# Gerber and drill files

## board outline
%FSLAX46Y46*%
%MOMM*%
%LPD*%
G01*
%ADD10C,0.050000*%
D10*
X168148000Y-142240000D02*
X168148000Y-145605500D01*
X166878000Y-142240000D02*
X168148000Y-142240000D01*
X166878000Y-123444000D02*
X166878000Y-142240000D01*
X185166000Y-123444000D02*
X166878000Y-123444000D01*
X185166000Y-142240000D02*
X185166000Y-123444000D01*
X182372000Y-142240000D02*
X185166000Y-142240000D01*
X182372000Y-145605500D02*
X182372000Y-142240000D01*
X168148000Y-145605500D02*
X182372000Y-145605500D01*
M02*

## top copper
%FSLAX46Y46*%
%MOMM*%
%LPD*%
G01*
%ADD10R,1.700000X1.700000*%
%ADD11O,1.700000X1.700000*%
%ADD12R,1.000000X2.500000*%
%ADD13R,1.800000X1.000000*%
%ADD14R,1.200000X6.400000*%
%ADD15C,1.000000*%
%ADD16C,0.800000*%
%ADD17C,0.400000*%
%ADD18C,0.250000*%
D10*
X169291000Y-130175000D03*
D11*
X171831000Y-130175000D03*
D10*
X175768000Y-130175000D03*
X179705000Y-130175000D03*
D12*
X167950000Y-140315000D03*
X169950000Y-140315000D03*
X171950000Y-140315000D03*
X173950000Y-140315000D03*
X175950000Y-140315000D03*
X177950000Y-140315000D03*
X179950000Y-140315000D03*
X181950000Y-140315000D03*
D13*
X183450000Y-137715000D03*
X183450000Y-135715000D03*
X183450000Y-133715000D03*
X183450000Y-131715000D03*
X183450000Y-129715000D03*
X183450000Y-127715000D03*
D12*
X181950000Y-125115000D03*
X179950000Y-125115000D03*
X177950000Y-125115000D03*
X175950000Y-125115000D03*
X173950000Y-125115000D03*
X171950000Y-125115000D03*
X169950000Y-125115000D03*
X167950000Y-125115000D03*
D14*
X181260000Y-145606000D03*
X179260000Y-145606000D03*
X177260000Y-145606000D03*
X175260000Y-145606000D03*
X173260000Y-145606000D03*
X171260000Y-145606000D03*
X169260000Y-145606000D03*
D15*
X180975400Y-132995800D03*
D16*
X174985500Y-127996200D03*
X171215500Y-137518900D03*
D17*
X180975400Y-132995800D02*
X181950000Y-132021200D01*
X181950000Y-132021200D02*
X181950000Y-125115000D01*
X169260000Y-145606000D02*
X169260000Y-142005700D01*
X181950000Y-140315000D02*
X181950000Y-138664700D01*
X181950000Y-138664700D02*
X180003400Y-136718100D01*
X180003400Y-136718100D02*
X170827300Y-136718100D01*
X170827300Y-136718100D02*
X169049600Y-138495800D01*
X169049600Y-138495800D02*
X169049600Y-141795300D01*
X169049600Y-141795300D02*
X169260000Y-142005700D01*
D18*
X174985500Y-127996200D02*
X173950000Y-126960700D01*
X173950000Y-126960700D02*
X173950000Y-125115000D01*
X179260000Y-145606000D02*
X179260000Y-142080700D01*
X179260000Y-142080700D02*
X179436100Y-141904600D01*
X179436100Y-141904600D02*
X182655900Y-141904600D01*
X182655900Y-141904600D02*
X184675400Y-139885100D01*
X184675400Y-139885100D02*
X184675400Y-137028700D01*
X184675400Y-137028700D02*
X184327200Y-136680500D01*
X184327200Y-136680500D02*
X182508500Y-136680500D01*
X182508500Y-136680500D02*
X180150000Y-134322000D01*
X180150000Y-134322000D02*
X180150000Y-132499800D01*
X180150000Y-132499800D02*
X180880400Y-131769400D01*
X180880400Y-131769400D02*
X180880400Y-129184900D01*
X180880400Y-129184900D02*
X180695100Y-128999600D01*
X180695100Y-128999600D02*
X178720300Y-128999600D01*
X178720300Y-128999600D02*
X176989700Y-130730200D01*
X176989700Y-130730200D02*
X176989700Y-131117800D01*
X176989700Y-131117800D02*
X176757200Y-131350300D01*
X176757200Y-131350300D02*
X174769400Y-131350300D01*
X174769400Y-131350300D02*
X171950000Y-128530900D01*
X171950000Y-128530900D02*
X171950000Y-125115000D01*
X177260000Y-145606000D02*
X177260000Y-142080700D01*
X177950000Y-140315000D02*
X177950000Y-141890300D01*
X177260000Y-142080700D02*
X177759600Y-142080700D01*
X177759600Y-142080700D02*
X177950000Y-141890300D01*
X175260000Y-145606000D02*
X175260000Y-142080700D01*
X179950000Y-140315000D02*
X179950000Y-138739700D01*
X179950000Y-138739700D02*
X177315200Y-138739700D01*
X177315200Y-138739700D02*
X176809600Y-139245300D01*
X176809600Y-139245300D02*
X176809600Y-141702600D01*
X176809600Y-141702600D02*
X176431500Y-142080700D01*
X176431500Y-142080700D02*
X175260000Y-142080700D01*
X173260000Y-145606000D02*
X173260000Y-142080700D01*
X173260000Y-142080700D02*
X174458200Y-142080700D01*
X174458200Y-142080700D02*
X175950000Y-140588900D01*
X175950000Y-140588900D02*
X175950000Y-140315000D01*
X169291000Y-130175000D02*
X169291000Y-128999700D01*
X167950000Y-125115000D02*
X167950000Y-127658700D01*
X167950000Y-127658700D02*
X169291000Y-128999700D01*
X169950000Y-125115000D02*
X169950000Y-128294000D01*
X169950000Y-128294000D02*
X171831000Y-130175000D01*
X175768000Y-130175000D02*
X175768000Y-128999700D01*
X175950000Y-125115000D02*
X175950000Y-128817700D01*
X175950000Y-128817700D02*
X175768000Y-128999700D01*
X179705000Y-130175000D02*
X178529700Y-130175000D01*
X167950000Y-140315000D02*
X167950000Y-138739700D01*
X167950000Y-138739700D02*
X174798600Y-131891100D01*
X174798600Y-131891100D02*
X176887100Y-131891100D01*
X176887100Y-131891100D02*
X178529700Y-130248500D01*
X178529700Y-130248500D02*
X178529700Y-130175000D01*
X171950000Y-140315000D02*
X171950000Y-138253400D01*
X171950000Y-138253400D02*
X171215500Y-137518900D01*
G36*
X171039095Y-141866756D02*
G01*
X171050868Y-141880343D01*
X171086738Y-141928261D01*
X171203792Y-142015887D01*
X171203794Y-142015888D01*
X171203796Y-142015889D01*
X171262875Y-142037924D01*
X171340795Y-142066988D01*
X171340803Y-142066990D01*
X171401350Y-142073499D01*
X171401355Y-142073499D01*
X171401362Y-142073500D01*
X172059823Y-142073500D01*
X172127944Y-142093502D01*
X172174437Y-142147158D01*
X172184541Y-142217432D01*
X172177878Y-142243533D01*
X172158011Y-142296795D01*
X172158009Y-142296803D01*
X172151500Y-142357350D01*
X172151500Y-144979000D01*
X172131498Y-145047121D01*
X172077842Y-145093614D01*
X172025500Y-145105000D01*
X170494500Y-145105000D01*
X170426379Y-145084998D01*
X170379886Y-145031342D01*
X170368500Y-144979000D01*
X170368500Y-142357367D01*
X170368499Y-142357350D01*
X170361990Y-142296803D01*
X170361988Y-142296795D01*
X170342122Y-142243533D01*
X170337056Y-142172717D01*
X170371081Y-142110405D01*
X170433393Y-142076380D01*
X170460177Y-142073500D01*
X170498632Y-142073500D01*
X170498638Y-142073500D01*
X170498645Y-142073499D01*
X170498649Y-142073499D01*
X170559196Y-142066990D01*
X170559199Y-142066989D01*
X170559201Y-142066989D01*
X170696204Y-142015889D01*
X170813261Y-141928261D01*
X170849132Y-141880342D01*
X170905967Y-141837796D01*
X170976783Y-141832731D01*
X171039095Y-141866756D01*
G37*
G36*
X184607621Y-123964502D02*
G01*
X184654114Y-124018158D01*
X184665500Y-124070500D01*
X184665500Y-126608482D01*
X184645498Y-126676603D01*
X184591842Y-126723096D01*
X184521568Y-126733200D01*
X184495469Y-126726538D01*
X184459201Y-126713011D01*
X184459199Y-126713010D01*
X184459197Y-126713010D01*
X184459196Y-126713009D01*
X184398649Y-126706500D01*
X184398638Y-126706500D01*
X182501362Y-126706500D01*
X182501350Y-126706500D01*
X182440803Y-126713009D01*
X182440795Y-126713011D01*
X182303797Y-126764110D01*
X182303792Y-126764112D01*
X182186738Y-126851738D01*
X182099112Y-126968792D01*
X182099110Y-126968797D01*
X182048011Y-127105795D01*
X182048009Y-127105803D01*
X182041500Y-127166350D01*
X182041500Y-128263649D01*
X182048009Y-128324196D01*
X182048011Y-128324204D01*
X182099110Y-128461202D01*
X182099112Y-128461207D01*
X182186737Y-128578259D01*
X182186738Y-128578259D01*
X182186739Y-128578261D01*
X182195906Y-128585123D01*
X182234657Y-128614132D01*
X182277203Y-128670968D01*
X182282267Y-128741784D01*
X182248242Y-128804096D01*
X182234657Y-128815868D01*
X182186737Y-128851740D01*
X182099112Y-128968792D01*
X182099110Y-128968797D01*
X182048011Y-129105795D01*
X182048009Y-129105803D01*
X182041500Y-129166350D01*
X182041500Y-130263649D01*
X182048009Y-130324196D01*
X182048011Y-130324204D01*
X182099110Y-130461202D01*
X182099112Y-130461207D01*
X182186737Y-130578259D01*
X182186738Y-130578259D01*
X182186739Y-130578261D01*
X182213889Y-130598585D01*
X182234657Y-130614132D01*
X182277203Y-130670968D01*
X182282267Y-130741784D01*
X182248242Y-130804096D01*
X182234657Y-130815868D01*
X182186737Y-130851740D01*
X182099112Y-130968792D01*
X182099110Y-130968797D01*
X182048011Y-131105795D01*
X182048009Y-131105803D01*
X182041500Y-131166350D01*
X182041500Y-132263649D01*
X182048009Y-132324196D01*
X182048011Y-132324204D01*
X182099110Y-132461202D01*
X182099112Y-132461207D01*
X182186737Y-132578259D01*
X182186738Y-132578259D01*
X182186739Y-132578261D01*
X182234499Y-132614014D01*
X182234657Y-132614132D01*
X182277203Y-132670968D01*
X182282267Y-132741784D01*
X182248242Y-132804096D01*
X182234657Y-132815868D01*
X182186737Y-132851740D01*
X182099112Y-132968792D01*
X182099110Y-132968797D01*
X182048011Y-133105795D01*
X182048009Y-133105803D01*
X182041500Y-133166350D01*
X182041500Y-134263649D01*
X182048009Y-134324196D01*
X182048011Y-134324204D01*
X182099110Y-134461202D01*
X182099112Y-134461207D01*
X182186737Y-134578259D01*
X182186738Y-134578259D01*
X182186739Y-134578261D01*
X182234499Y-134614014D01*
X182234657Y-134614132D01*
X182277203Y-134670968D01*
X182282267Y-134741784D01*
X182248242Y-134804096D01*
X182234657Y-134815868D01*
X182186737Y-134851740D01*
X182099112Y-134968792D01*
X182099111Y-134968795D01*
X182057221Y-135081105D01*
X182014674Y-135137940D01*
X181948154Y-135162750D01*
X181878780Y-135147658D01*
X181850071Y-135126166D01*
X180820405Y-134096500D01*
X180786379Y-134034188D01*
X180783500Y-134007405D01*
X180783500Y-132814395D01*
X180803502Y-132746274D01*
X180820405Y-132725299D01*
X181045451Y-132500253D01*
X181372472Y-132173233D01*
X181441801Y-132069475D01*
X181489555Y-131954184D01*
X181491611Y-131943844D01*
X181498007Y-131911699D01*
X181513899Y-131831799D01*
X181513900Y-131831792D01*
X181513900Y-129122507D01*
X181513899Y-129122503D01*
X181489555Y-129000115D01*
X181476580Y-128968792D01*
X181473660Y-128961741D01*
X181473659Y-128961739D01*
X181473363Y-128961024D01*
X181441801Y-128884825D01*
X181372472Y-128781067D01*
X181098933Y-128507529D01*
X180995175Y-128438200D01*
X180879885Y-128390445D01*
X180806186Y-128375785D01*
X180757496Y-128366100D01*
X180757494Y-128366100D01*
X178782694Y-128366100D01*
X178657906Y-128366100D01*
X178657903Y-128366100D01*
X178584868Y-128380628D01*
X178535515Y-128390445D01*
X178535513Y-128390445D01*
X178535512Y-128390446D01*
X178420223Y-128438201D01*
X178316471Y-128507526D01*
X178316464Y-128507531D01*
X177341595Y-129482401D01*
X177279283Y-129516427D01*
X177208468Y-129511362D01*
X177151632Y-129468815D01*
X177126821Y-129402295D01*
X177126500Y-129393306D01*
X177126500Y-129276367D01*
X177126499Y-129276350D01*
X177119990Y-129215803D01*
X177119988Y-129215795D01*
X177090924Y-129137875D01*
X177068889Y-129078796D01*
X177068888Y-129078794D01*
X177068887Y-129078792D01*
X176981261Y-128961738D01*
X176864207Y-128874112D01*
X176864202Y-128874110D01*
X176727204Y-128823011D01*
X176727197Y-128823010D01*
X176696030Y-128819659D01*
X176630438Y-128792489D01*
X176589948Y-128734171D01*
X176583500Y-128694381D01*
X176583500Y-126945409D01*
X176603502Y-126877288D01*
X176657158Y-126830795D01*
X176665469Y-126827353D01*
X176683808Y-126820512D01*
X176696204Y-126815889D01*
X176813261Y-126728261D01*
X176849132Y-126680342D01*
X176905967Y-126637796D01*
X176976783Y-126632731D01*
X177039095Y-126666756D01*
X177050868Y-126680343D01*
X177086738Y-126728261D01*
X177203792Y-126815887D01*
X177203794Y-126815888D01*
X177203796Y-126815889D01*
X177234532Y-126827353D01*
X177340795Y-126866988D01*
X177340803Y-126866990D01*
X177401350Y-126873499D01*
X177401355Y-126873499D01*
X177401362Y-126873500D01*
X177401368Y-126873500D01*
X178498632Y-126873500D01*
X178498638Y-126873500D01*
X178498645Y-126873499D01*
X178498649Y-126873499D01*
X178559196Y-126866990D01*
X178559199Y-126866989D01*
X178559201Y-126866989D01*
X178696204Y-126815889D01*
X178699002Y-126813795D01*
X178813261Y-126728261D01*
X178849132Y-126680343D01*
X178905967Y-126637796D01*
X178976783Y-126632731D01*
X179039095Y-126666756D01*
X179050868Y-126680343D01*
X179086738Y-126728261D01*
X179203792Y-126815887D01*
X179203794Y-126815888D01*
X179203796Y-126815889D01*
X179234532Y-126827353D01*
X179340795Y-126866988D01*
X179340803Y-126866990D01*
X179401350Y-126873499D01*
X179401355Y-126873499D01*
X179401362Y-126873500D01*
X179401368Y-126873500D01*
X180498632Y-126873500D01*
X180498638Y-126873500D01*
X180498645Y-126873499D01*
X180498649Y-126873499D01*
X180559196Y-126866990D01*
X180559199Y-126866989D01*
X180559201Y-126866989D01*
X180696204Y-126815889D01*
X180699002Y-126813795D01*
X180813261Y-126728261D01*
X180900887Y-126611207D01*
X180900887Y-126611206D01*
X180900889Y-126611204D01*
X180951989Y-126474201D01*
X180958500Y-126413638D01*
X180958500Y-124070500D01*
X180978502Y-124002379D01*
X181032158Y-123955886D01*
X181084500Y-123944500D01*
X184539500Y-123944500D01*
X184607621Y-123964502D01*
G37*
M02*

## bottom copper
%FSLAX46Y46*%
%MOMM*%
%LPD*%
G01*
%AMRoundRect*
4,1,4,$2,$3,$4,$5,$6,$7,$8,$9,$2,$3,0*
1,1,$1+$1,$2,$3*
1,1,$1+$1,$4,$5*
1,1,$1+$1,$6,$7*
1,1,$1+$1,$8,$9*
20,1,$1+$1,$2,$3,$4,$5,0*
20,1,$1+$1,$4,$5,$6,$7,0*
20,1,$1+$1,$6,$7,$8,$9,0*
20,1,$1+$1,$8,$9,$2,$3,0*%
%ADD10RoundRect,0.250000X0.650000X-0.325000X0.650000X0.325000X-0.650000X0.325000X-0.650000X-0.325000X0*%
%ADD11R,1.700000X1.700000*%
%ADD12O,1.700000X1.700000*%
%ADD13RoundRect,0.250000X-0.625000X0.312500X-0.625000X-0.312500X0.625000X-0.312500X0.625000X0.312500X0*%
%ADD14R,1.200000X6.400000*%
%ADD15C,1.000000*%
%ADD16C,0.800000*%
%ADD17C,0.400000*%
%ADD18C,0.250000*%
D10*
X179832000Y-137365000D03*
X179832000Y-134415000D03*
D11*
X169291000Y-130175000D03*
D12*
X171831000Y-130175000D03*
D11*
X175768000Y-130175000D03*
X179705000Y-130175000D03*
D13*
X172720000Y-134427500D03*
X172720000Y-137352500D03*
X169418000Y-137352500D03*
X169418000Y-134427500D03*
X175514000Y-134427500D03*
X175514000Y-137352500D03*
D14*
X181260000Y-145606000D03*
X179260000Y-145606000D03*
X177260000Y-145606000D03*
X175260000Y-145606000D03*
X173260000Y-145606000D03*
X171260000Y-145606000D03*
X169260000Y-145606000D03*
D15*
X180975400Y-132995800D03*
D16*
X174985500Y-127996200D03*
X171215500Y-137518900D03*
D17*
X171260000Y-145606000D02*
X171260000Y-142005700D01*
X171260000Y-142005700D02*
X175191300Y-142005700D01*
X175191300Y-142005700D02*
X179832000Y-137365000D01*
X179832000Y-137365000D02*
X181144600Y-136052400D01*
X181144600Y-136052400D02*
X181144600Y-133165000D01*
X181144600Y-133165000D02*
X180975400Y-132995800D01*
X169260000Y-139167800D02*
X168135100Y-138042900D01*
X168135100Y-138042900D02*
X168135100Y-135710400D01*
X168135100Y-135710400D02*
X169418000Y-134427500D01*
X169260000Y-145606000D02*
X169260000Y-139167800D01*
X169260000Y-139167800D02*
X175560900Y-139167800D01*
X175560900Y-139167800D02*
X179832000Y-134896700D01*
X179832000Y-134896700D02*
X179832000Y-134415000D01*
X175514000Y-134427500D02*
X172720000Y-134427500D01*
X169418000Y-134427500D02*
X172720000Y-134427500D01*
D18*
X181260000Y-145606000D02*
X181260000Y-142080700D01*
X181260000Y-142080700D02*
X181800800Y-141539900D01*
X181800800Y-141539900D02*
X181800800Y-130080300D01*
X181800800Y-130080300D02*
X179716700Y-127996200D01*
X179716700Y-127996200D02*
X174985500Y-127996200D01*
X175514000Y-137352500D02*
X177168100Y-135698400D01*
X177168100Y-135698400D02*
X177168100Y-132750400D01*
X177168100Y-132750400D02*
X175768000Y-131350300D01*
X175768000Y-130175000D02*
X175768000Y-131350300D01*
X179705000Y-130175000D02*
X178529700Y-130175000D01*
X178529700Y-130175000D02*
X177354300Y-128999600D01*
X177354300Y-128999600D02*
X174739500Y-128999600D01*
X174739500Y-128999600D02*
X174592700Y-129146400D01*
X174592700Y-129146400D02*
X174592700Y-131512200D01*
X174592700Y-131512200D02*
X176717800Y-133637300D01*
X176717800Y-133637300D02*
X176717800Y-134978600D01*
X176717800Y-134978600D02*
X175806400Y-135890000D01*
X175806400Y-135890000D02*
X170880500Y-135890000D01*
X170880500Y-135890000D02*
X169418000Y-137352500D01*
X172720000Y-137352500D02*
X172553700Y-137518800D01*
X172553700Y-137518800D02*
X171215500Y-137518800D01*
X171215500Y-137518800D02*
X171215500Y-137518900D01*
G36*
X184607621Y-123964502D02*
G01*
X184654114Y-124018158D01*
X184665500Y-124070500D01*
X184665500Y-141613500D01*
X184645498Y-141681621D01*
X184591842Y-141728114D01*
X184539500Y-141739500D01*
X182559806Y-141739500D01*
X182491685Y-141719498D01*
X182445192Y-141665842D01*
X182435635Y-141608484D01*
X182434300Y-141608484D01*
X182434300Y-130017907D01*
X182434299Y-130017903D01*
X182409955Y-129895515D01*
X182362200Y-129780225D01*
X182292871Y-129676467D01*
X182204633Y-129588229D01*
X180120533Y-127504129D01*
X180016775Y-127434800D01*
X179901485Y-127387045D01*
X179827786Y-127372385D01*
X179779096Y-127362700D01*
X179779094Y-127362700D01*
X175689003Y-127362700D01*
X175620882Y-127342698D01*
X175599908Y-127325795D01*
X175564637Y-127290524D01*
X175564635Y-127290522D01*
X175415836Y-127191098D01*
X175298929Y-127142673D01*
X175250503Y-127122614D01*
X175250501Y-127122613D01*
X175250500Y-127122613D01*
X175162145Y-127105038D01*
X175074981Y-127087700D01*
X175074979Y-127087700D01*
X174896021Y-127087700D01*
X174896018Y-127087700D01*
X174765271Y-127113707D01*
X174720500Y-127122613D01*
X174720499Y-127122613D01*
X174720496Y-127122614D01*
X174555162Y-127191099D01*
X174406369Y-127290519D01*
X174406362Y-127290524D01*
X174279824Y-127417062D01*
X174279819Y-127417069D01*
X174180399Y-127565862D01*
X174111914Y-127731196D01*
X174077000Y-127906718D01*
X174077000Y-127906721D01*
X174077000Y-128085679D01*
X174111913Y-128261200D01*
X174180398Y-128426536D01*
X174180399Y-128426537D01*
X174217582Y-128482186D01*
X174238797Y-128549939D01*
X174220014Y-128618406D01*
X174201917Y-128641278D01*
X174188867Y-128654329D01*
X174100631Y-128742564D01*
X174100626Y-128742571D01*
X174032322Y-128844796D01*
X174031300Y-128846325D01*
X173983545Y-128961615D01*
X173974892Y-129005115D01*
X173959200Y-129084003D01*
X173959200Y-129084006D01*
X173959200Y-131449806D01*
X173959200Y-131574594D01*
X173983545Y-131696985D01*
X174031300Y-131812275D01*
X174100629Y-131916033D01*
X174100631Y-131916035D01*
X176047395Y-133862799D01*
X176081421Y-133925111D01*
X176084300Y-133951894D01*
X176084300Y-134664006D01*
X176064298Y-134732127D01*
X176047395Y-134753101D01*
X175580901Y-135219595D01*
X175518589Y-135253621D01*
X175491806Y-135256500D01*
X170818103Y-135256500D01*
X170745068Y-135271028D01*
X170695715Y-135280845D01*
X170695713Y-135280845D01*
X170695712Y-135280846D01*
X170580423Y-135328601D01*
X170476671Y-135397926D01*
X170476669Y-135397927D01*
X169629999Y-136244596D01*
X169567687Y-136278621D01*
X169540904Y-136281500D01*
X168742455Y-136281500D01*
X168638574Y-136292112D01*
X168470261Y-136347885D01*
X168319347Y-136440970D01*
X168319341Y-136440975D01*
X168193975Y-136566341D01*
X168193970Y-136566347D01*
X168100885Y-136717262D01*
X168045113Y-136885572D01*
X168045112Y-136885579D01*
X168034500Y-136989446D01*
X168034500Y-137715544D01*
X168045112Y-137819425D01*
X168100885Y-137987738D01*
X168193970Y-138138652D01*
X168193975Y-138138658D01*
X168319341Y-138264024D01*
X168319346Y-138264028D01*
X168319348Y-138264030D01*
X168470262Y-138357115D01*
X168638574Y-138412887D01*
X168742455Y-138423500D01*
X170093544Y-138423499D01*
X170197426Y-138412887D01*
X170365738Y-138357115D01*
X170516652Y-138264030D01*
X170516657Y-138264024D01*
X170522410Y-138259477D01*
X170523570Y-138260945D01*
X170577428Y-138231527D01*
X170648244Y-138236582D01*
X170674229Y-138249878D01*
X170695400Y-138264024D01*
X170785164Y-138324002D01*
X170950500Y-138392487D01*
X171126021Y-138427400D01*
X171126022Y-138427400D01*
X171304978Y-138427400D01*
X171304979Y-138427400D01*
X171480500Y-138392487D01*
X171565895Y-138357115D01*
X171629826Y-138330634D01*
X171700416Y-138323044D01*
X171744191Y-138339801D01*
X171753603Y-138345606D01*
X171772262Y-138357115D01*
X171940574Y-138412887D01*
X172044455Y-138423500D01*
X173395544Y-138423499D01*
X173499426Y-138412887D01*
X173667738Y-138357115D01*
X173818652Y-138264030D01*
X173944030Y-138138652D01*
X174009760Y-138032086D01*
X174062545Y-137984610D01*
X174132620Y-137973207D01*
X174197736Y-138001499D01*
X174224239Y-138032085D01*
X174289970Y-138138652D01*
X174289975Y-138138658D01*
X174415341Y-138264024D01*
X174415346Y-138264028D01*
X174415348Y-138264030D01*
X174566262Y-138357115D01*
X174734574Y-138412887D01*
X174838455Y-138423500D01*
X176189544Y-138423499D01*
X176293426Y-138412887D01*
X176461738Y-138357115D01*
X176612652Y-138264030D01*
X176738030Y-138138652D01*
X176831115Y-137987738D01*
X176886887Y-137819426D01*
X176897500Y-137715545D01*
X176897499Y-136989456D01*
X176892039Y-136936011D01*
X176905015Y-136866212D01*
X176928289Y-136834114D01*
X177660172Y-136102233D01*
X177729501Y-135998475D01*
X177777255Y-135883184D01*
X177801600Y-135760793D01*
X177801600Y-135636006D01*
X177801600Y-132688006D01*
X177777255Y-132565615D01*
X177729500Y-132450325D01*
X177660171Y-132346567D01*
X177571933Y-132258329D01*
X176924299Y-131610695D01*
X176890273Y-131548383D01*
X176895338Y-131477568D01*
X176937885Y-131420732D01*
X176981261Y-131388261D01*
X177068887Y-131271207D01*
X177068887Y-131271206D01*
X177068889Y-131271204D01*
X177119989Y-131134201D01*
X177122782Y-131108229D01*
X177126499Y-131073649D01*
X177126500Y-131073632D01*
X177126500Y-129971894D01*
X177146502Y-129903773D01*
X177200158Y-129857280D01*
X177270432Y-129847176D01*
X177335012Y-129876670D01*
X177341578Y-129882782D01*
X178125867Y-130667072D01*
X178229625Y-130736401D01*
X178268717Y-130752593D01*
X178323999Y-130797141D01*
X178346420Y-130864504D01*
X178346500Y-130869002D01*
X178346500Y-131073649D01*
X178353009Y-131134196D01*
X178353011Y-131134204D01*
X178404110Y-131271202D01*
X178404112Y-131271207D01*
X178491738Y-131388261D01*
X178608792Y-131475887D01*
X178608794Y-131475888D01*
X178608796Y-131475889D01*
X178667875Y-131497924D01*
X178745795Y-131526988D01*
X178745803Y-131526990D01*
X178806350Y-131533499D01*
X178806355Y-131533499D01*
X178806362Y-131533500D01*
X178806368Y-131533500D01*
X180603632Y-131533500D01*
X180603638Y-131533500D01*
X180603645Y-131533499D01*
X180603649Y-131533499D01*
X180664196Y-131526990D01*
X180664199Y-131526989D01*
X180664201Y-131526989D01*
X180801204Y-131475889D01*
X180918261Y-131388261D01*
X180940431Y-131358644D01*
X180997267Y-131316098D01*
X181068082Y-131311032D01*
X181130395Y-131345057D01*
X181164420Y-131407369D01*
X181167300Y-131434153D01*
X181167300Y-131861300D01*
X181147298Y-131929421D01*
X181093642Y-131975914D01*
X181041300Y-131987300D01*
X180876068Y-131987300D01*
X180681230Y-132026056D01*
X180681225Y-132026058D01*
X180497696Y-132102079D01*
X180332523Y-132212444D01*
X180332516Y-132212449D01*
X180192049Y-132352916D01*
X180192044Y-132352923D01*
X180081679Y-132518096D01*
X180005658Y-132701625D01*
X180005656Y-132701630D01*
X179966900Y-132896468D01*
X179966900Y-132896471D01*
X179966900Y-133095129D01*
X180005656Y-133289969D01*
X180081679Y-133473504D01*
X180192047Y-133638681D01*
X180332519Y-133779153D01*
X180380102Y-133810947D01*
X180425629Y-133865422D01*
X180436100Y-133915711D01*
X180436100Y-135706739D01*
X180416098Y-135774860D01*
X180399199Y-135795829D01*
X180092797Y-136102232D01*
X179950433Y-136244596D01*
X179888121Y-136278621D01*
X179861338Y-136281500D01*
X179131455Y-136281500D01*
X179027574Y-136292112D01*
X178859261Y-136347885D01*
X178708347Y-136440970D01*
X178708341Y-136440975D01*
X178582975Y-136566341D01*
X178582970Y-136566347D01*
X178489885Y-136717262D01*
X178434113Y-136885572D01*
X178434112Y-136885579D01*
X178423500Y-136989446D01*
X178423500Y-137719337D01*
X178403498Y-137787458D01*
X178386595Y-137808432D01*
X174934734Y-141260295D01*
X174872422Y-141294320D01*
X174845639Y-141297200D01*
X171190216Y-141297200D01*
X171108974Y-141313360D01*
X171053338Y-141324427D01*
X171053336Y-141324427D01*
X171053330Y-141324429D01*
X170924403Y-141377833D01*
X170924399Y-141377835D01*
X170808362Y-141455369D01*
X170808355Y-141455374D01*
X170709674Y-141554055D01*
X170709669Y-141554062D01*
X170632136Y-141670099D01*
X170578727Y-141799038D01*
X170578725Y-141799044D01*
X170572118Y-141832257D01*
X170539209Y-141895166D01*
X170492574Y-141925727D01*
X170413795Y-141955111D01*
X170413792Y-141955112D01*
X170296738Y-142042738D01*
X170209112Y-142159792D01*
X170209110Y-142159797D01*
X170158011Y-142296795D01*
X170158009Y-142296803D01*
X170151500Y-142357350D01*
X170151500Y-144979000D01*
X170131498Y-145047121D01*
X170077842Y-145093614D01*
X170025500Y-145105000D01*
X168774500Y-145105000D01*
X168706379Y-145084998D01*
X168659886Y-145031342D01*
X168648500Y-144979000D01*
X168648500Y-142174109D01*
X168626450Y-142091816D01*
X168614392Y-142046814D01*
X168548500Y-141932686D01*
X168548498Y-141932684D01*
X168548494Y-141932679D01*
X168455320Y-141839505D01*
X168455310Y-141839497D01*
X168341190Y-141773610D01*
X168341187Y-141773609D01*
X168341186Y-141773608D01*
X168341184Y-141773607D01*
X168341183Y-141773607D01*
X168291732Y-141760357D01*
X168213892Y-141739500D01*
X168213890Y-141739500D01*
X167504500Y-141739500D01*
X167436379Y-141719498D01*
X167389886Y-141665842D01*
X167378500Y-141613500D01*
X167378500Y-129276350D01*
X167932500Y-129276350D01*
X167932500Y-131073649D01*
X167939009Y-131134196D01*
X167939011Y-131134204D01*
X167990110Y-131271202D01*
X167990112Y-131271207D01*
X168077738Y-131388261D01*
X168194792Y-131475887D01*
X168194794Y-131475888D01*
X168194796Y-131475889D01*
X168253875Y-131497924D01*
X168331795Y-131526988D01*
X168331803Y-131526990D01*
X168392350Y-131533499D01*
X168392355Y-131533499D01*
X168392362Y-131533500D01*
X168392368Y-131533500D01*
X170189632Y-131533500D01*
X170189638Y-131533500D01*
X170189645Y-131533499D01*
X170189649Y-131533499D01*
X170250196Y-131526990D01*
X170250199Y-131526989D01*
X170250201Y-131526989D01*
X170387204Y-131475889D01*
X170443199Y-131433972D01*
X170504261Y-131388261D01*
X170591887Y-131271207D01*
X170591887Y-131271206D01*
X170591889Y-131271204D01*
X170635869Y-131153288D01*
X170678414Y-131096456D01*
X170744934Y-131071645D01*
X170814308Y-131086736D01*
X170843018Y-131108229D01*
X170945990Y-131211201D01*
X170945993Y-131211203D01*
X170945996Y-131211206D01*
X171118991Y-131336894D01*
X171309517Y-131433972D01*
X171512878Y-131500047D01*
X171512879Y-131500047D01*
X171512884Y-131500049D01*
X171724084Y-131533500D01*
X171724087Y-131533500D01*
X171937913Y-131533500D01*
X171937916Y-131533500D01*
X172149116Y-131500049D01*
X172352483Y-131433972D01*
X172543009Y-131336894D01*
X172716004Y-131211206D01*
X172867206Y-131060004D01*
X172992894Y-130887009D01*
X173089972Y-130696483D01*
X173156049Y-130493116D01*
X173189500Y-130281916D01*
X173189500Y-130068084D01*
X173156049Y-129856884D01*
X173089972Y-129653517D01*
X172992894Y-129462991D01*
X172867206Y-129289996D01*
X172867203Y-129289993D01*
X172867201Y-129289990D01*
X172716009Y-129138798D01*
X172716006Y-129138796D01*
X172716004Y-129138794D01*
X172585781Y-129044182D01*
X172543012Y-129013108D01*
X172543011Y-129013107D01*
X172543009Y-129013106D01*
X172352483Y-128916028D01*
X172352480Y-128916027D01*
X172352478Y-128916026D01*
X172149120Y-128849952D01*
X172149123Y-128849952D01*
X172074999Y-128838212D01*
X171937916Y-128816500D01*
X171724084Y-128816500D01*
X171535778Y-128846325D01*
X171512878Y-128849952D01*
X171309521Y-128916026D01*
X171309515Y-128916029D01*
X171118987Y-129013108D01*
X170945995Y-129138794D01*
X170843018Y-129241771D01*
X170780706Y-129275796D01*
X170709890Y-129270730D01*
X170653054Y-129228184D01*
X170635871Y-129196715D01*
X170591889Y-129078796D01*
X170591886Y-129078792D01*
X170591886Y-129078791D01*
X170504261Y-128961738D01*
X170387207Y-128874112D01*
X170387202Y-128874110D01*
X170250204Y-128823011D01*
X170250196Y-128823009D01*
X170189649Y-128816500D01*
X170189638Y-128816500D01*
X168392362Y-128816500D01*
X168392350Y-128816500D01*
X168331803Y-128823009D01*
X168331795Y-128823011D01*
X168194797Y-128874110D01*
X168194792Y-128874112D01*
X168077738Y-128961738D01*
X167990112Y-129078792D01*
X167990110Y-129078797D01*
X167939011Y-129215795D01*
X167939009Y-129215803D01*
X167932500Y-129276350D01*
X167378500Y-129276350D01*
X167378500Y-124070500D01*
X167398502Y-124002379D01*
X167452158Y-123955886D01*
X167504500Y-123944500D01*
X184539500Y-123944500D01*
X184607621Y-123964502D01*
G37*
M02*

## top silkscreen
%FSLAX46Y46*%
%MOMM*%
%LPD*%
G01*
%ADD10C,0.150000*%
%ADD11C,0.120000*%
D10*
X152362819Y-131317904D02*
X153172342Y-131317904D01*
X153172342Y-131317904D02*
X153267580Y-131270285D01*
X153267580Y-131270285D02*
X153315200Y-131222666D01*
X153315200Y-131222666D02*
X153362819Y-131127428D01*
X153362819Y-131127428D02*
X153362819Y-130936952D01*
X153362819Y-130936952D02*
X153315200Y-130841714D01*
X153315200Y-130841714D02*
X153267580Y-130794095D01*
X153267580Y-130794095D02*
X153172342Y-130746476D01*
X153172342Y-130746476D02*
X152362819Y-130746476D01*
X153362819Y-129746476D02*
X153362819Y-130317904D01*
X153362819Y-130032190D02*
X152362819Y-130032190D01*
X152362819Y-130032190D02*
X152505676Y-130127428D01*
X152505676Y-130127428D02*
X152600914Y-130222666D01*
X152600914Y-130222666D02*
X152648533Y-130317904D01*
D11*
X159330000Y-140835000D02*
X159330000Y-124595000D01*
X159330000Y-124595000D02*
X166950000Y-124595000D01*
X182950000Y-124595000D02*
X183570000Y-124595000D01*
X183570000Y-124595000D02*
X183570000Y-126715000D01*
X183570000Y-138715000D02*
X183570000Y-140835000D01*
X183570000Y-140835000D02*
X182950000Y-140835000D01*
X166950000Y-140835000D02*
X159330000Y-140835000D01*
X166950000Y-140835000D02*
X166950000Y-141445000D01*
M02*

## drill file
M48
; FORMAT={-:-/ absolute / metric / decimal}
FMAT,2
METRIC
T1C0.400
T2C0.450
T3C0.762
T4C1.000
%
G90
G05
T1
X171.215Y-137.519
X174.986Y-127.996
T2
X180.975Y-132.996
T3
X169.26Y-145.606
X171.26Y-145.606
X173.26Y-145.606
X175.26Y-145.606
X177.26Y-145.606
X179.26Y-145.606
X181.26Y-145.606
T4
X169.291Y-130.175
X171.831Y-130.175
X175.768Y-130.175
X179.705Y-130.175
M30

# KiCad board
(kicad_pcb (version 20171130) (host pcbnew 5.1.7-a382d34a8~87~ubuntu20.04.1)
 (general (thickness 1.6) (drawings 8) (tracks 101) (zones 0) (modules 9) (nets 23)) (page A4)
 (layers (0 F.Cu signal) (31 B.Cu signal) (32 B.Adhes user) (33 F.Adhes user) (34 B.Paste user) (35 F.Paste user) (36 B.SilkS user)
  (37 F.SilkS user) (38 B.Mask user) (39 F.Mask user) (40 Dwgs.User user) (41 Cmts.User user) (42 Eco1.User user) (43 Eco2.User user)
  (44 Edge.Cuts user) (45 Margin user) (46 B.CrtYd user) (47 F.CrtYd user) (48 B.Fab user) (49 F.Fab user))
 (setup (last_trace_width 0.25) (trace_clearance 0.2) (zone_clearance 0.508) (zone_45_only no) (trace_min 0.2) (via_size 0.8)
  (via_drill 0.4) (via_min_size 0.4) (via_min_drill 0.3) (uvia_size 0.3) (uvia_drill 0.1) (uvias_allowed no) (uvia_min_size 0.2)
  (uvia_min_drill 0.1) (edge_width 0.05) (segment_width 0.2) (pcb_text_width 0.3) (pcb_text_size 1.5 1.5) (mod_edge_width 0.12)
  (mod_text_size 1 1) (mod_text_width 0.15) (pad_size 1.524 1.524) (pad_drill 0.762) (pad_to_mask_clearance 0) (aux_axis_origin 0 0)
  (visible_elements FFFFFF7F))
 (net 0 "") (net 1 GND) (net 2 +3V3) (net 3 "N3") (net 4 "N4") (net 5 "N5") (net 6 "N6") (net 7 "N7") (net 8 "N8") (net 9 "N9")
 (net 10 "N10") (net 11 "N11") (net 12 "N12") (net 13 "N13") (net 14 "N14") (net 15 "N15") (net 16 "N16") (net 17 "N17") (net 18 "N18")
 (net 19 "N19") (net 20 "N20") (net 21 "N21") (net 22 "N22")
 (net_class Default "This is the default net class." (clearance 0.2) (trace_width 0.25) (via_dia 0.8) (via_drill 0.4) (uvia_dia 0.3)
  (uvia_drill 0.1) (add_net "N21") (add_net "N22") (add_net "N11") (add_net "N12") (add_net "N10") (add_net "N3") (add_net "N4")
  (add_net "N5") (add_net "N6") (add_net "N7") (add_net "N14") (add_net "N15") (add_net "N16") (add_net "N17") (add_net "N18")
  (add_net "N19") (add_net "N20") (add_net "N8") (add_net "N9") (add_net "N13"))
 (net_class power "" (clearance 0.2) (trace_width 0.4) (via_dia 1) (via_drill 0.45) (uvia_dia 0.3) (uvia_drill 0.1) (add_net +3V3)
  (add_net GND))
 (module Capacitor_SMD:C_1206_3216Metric (layer B.Cu) (at 179.832 135.89 90)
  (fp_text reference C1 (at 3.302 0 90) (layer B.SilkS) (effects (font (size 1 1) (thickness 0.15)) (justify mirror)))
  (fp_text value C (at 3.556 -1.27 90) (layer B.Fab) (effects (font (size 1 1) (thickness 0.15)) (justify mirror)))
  (pad 1 smd roundrect (at -1.475 0 90) (size 1.15 1.8) (layers B.Cu B.Paste B.Mask) (roundrect_rratio 0.217391) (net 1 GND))
  (pad 2 smd roundrect (at 1.475 0 90) (size 1.15 1.8) (layers B.Cu B.Paste B.Mask) (roundrect_rratio 0.217391) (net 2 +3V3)))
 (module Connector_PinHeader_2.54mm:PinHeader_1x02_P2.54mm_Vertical (layer B.Cu) (at 169.291 130.175 270)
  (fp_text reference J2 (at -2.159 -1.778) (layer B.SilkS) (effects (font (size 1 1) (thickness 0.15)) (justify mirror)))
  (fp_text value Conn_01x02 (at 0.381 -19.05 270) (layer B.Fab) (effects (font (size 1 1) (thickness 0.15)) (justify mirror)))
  (pad 1 thru_hole rect (at 0 0 270) (size 1.7 1.7) (drill 1) (layers *.Cu *.Mask) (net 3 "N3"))
  (pad 2 thru_hole oval (at 0 -2.54 270) (size 1.7 1.7) (drill 1) (layers *.Cu *.Mask) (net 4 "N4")))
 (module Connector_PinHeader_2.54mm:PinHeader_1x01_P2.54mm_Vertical (layer B.Cu) (at 175.768 130.175)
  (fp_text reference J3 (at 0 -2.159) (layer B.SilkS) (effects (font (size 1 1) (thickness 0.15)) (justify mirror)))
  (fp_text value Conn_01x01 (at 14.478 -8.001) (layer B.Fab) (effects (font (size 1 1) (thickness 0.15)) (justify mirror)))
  (pad 1 thru_hole rect (at 0 0) (size 1.7 1.7) (drill 1) (layers *.Cu *.Mask) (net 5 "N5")))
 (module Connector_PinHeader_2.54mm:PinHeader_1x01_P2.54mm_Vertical (layer B.Cu) (at 179.705 130.175)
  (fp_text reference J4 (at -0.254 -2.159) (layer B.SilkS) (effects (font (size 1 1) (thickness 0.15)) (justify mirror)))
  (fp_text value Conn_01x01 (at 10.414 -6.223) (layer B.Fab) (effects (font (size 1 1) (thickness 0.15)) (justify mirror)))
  (pad 1 thru_hole rect (at 0 0) (size 1.7 1.7) (drill 1) (layers *.Cu *.Mask) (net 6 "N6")))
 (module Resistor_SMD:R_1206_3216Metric (layer B.Cu) (at 172.72 135.89 270)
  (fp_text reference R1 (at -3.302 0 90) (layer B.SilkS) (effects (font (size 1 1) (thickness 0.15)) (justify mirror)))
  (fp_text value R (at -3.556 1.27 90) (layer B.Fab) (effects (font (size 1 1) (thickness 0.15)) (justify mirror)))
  (pad 1 smd roundrect (at -1.4625 0 270) (size 1.125 1.75) (layers B.Cu B.Paste B.Mask) (roundrect_rratio 0.222222) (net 2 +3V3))
  (pad 2 smd roundrect (at 1.4625 0 270) (size 1.125 1.75) (layers B.Cu B.Paste B.Mask) (roundrect_rratio 0.222222) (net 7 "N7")))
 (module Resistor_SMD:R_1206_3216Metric (layer B.Cu) (at 169.418 135.89 270)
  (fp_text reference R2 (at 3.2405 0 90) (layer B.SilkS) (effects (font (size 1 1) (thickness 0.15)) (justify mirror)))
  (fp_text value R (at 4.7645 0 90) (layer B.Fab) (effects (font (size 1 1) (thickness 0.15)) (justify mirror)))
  (pad 2 smd roundrect (at 1.4625 0 270) (size 1.125 1.75) (layers B.Cu B.Paste B.Mask) (roundrect_rratio 0.222222) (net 6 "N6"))
  (pad 1 smd roundrect (at -1.4625 0 270) (size 1.125 1.75) (layers B.Cu B.Paste B.Mask) (roundrect_rratio 0.222222) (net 2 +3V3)))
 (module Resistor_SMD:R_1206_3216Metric (layer B.Cu) (at 175.514 135.89 270)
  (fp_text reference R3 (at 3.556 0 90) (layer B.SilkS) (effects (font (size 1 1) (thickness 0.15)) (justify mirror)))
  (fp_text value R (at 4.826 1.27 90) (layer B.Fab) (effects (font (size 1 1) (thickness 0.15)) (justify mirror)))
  (pad 1 smd roundrect (at -1.4625 0 270) (size 1.125 1.75) (layers B.Cu B.Paste B.Mask) (roundrect_rratio 0.222222) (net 2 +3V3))
  (pad 2 smd roundrect (at 1.4625 0 270) (size 1.125 1.75) (layers B.Cu B.Paste B.Mask) (roundrect_rratio 0.222222) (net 5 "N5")))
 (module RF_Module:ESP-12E (layer F.Cu) (at 171.45 132.715 90)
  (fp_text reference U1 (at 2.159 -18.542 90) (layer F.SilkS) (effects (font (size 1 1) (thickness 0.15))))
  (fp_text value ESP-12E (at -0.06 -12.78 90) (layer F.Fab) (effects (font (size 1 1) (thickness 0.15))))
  (fp_line (start -8.12 -12.12) (end 8.12 -12.12) (layer F.SilkS) (width 0.12))
  (fp_line (start 8.12 -12.12) (end 8.12 -4.5) (layer F.SilkS) (width 0.12))
  (fp_line (start 8.12 11.5) (end 8.12 12.12) (layer F.SilkS) (width 0.12))
  (fp_line (start 8.12 12.12) (end 6 12.12) (layer F.SilkS) (width 0.12))
  (fp_line (start -6 12.12) (end -8.12 12.12) (layer F.SilkS) (width 0.12))
  (fp_line (start -8.12 12.12) (end -8.12 11.5) (layer F.SilkS) (width 0.12))
  (fp_line (start -8.12 -4.5) (end -8.12 -12.12) (layer F.SilkS) (width 0.12))
  (fp_line (start -8.12 -4.5) (end -8.73 -4.5) (layer F.SilkS) (width 0.12))
  (pad 1 smd rect (at -7.6 -3.5 90) (size 2.5 1) (layers F.Cu F.Paste F.Mask) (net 6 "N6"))
  (pad 2 smd rect (at -7.6 -1.5 90) (size 2.5 1) (layers F.Cu F.Paste F.Mask) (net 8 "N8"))
  (pad 3 smd rect (at -7.6 0.5 90) (size 2.5 1) (layers F.Cu F.Paste F.Mask) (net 7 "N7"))
  (pad 4 smd rect (at -7.6 2.5 90) (size 2.5 1) (layers F.Cu F.Paste F.Mask) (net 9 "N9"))
  (pad 5 smd rect (at -7.6 4.5 90) (size 2.5 1) (layers F.Cu F.Paste F.Mask) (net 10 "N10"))
  (pad 6 smd rect (at -7.6 6.5 90) (size 2.5 1) (layers F.Cu F.Paste F.Mask) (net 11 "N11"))
  (pad 7 smd rect (at -7.6 8.5 90) (size 2.5 1) (layers F.Cu F.Paste F.Mask) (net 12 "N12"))
  (pad 8 smd rect (at -7.6 10.5 90) (size 2.5 1) (layers F.Cu F.Paste F.Mask) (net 2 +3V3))
  (pad 9 smd rect (at -5 12 90) (size 1 1.8) (layers F.Cu F.Paste F.Mask) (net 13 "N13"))
  (pad 10 smd rect (at -3 12 90) (size 1 1.8) (layers F.Cu F.Paste F.Mask) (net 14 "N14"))
  (pad 11 smd rect (at -1 12 90) (size 1 1.8) (layers F.Cu F.Paste F.Mask) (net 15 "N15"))
  (pad 12 smd rect (at 1 12 90) (size 1 1.8) (layers F.Cu F.Paste F.Mask) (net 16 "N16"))
  (pad 13 smd rect (at 3 12 90) (size 1 1.8) (layers F.Cu F.Paste F.Mask) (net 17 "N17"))
  (pad 14 smd rect (at 5 12 90) (size 1 1.8) (layers F.Cu F.Paste F.Mask) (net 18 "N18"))
  (pad 15 smd rect (at 7.6 10.5 90) (size 2.5 1) (layers F.Cu F.Paste F.Mask) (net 1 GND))
  (pad 16 smd rect (at 7.6 8.5 90) (size 2.5 1) (layers F.Cu F.Paste F.Mask) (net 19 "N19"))
  (pad 17 smd rect (at 7.6 6.5 90) (size 2.5 1) (layers F.Cu F.Paste F.Mask) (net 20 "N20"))
  (pad 18 smd rect (at 7.6 4.5 90) (size 2.5 1) (layers F.Cu F.Paste F.Mask) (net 5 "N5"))
  (pad 19 smd rect (at 7.6 2.5 90) (size 2.5 1) (layers F.Cu F.Paste F.Mask) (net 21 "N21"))
  (pad 20 smd rect (at 7.6 0.5 90) (size 2.5 1) (layers F.Cu F.Paste F.Mask) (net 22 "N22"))
  (pad 21 smd rect (at 7.6 -1.5 90) (size 2.5 1) (layers F.Cu F.Paste F.Mask) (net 4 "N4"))
  (pad 22 smd rect (at 7.6 -3.5 90) (size 2.5 1) (layers F.Cu F.Paste F.Mask) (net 3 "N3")))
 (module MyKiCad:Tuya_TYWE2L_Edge (layer B.Cu) (at 175.26 135.606 180)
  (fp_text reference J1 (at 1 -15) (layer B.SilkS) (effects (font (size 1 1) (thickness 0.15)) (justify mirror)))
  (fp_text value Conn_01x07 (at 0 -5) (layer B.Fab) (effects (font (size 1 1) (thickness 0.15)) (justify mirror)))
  (pad 1 thru_hole rect (at -6 -10 180) (size 1.2 6.4) (drill 0.762) (layers *.Cu *.Mask) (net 21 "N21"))
  (pad 2 thru_hole rect (at -4 -10 180) (size 1.2 6.4) (drill 0.762) (layers *.Cu *.Mask) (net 22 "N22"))
  (pad 3 thru_hole rect (at -2 -10 180) (size 1.2 6.4) (drill 0.762) (layers *.Cu *.Mask) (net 11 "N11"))
  (pad 4 thru_hole rect (at 0 -10 180) (size 1.2 6.4) (drill 0.762) (layers *.Cu *.Mask) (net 12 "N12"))
  (pad 5 thru_hole rect (at 2 -10 180) (size 1.2 6.4) (drill 0.762) (layers *.Cu *.Mask) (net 10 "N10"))
  (pad 6 thru_hole rect (at 4 -10 180) (size 1.2 6.4) (drill 0.762) (layers *.Cu *.Mask) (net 1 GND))
  (pad 7 thru_hole rect (at 6 -10 180) (size 1.2 6.4) (drill 0.762) (layers *.Cu *.Mask) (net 2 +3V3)))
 (gr_line (start 168.148 142.24) (end 168.148 145.6055) (layer Edge.Cuts) (width 0.05))
 (gr_line (start 166.878 142.24) (end 168.148 142.24) (layer Edge.Cuts) (width 0.05))
 (gr_line (start 166.878 123.444) (end 166.878 142.24) (layer Edge.Cuts) (width 0.05))
 (gr_line (start 185.166 123.444) (end 166.878 123.444) (layer Edge.Cuts) (width 0.05))
 (gr_line (start 185.166 142.24) (end 185.166 123.444) (layer Edge.Cuts) (width 0.05))
 (gr_line (start 182.372 142.24) (end 185.166 142.24) (layer Edge.Cuts) (width 0.05))
 (gr_line (start 182.372 145.6055) (end 182.372 142.24) (layer Edge.Cuts) (width 0.05))
 (gr_line (start 168.148 145.6055) (end 182.372 145.6055) (layer Edge.Cuts) (width 0.05))
 (segment (start 171.26 145.606) (end 171.26 142.0057) (width 0.4) (layer B.Cu) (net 1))
 (segment (start 171.26 142.0057) (end 175.1913 142.0057) (width 0.4) (layer B.Cu) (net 1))
 (segment (start 175.1913 142.0057) (end 179.832 137.365) (width 0.4) (layer B.Cu) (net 1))
 (segment (start 180.9754 132.9958) (end 181.95 132.0212) (width 0.4) (layer F.Cu) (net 1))
 (segment (start 181.95 132.0212) (end 181.95 125.115) (width 0.4) (layer F.Cu) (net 1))
 (segment (start 179.832 137.365) (end 181.1446 136.0524) (width 0.4) (layer B.Cu) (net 1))
 (segment (start 181.1446 136.0524) (end 181.1446 133.165) (width 0.4) (layer B.Cu) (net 1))
 (segment (start 181.1446 133.165) (end 180.9754 132.9958) (width 0.4) (layer B.Cu) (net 1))
 (via (at 180.9754 132.9958) (size 1) (drill 0.45) (layers F.Cu B.Cu) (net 1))
 (segment (start 169.26 145.606) (end 169.26 142.0057) (width 0.4) (layer F.Cu) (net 2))
 (segment (start 181.95 140.315) (end 181.95 138.6647) (width 0.4) (layer F.Cu) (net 2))
 (segment (start 181.95 138.6647) (end 180.0034 136.7181) (width 0.4) (layer F.Cu) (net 2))
 (segment (start 180.0034 136.7181) (end 170.8273 136.7181) (width 0.4) (layer F.Cu) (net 2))
 (segment (start 170.8273 136.7181) (end 169.0496 138.4958) (width 0.4) (layer F.Cu) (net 2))
 (segment (start 169.0496 138.4958) (end 169.0496 141.7953) (width 0.4) (layer F.Cu) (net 2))
 (segment (start 169.0496 141.7953) (end 169.26 142.0057) (width 0.4) (layer F.Cu) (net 2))
 (segment (start 169.26 139.1678) (end 168.1351 138.0429) (width 0.4) (layer B.Cu) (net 2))
 (segment (start 168.1351 138.0429) (end 168.1351 135.7104) (width 0.4) (layer B.Cu) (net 2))
 (segment (start 168.1351 135.7104) (end 169.418 134.4275) (width 0.4) (layer B.Cu) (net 2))
 (segment (start 169.26 145.606) (end 169.26 139.1678) (width 0.4) (layer B.Cu) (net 2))
 (segment (start 169.26 139.1678) (end 175.5609 139.1678) (width 0.4) (layer B.Cu) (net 2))
 (segment (start 175.5609 139.1678) (end 179.832 134.8967) (width 0.4) (layer B.Cu) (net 2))
 (segment (start 179.832 134.8967) (end 179.832 134.415) (width 0.4) (layer B.Cu) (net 2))
 (segment (start 175.514 134.4275) (end 172.72 134.4275) (width 0.4) (layer B.Cu) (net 2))
 (segment (start 169.418 134.4275) (end 172.72 134.4275) (width 0.4) (layer B.Cu) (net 2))
 (segment (start 181.26 145.606) (end 181.26 142.0807) (width 0.25) (layer B.Cu) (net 21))
 (segment (start 174.9855 127.9962) (end 173.95 126.9607) (width 0.25) (layer F.Cu) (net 21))
 (segment (start 173.95 126.9607) (end 173.95 125.115) (width 0.25) (layer F.Cu) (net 21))
 (segment (start 181.26 142.0807) (end 181.8008 141.5399) (width 0.25) (layer B.Cu) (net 21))
 (segment (start 181.8008 141.5399) (end 181.8008 130.0803) (width 0.25) (layer B.Cu) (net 21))
 (segment (start 181.8008 130.0803) (end 179.7167 127.9962) (width 0.25) (layer B.Cu) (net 21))
 (segment (start 179.7167 127.9962) (end 174.9855 127.9962) (width 0.25) (layer B.Cu) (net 21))
 (via (at 174.9855 127.9962) (size 0.8) (layers F.Cu B.Cu) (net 21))
 (segment (start 179.26 145.606) (end 179.26 142.0807) (width 0.25) (layer F.Cu) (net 22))
 (segment (start 179.26 142.0807) (end 179.4361 141.9046) (width 0.25) (layer F.Cu) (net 22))
 (segment (start 179.4361 141.9046) (end 182.6559 141.9046) (width 0.25) (layer F.Cu) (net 22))
 (segment (start 182.6559 141.9046) (end 184.6754 139.8851) (width 0.25) (layer F.Cu) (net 22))
 (segment (start 184.6754 139.8851) (end 184.6754 137.0287) (width 0.25) (layer F.Cu) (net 22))
 (segment (start 184.6754 137.0287) (end 184.3272 136.6805) (width 0.25) (layer F.Cu) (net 22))
 (segment (start 184.3272 136.6805) (end 182.5085 136.6805) (width 0.25) (layer F.Cu) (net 22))
 (segment (start 182.5085 136.6805) (end 180.15 134.322) (width 0.25) (layer F.Cu) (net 22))
 (segment (start 180.15 134.322) (end 180.15 132.4998) (width 0.25) (layer F.Cu) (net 22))
 (segment (start 180.15 132.4998) (end 180.8804 131.7694) (width 0.25) (layer F.Cu) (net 22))
 (segment (start 180.8804 131.7694) (end 180.8804 129.1849) (width 0.25) (layer F.Cu) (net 22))
 (segment (start 180.8804 129.1849) (end 180.6951 128.9996) (width 0.25) (layer F.Cu) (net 22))
 (segment (start 180.6951 128.9996) (end 178.7203 128.9996) (width 0.25) (layer F.Cu) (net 22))
 (segment (start 178.7203 128.9996) (end 176.9897 130.7302) (width 0.25) (layer F.Cu) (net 22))
 (segment (start 176.9897 130.7302) (end 176.9897 131.1178) (width 0.25) (layer F.Cu) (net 22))
 (segment (start 176.9897 131.1178) (end 176.7572 131.3503) (width 0.25) (layer F.Cu) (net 22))
 (segment (start 176.7572 131.3503) (end 174.7694 131.3503) (width 0.25) (layer F.Cu) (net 22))
 (segment (start 174.7694 131.3503) (end 171.95 128.5309) (width 0.25) (layer F.Cu) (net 22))
 (segment (start 171.95 128.5309) (end 171.95 125.115) (width 0.25) (layer F.Cu) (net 22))
 (segment (start 177.26 145.606) (end 177.26 142.0807) (width 0.25) (layer F.Cu) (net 11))
 (segment (start 177.95 140.315) (end 177.95 141.8903) (width 0.25) (layer F.Cu) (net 11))
 (segment (start 177.26 142.0807) (end 177.7596 142.0807) (width 0.25) (layer F.Cu) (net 11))
 (segment (start 177.7596 142.0807) (end 177.95 141.8903) (width 0.25) (layer F.Cu) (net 11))
 (segment (start 175.26 145.606) (end 175.26 142.0807) (width 0.25) (layer F.Cu) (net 12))
 (segment (start 179.95 140.315) (end 179.95 138.7397) (width 0.25) (layer F.Cu) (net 12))
 (segment (start 179.95 138.7397) (end 177.3152 138.7397) (width 0.25) (layer F.Cu) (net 12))
 (segment (start 177.3152 138.7397) (end 176.8096 139.2453) (width 0.25) (layer F.Cu) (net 12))
 (segment (start 176.8096 139.2453) (end 176.8096 141.7026) (width 0.25) (layer F.Cu) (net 12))
 (segment (start 176.8096 141.7026) (end 176.4315 142.0807) (width 0.25) (layer F.Cu) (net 12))
 (segment (start 176.4315 142.0807) (end 175.26 142.0807) (width 0.25) (layer F.Cu) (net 12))
 (segment (start 173.26 145.606) (end 173.26 142.0807) (width 0.25) (layer F.Cu) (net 10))
 (segment (start 173.26 142.0807) (end 174.4582 142.0807) (width 0.25) (layer F.Cu) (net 10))
 (segment (start 174.4582 142.0807) (end 175.95 140.5889) (width 0.25) (layer F.Cu) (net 10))
 (segment (start 175.95 140.5889) (end 175.95 140.315) (width 0.25) (layer F.Cu) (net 10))
 (segment (start 169.291 130.175) (end 169.291 128.9997) (width 0.25) (layer F.Cu) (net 3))
 (segment (start 167.95 125.115) (end 167.95 127.6587) (width 0.25) (layer F.Cu) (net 3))
 (segment (start 167.95 127.6587) (end 169.291 128.9997) (width 0.25) (layer F.Cu) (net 3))
 (segment (start 169.95 125.115) (end 169.95 128.294) (width 0.25) (layer F.Cu) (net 4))
 (segment (start 169.95 128.294) (end 171.831 130.175) (width 0.25) (layer F.Cu) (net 4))
 (segment (start 175.514 137.3525) (end 177.1681 135.6984) (width 0.25) (layer B.Cu) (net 5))
 (segment (start 177.1681 135.6984) (end 177.1681 132.7504) (width 0.25) (layer B.Cu) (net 5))
 (segment (start 177.1681 132.7504) (end 175.768 131.3503) (width 0.25) (layer B.Cu) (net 5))
 (segment (start 175.768 130.175) (end 175.768 131.3503) (width 0.25) (layer B.Cu) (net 5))
 (segment (start 175.768 130.175) (end 175.768 128.9997) (width 0.25) (layer F.Cu) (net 5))
 (segment (start 175.95 125.115) (end 175.95 128.8177) (width 0.25) (layer F.Cu) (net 5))
 (segment (start 175.95 128.8177) (end 175.768 128.9997) (width 0.25) (layer F.Cu) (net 5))
 (segment (start 179.705 130.175) (end 178.5297 130.175) (width 0.25) (layer F.Cu) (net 6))
 (segment (start 167.95 140.315) (end 167.95 138.7397) (width 0.25) (layer F.Cu) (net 6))
 (segment (start 167.95 138.7397) (end 174.7986 131.8911) (width 0.25) (layer F.Cu) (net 6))
 (segment (start 174.7986 131.8911) (end 176.8871 131.8911) (width 0.25) (layer F.Cu) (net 6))
 (segment (start 176.8871 131.8911) (end 178.5297 130.2485) (width 0.25) (layer F.Cu) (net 6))
 (segment (start 178.5297 130.2485) (end 178.5297 130.175) (width 0.25) (layer F.Cu) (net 6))
 (segment (start 179.705 130.175) (end 178.5297 130.175) (width 0.25) (layer B.Cu) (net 6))
 (segment (start 178.5297 130.175) (end 177.3543 128.9996) (width 0.25) (layer B.Cu) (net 6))
 (segment (start 177.3543 128.9996) (end 174.7395 128.9996) (width 0.25) (layer B.Cu) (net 6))
 (segment (start 174.7395 128.9996) (end 174.5927 129.1464) (width 0.25) (layer B.Cu) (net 6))
 (segment (start 174.5927 129.1464) (end 174.5927 131.5122) (width 0.25) (layer B.Cu) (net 6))
 (segment (start 174.5927 131.5122) (end 176.7178 133.6373) (width 0.25) (layer B.Cu) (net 6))
 (segment (start 176.7178 133.6373) (end 176.7178 134.9786) (width 0.25) (layer B.Cu) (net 6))
 (segment (start 176.7178 134.9786) (end 175.8064 135.89) (width 0.25) (layer B.Cu) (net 6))
 (segment (start 175.8064 135.89) (end 170.8805 135.89) (width 0.25) (layer B.Cu) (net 6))
 (segment (start 170.8805 135.89) (end 169.418 137.3525) (width 0.25) (layer B.Cu) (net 6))
 (segment (start 171.95 140.315) (end 171.95 138.2534) (width 0.25) (layer F.Cu) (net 7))
 (segment (start 171.95 138.2534) (end 171.2155 137.5189) (width 0.25) (layer F.Cu) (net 7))
 (segment (start 172.72 137.3525) (end 172.5537 137.5188) (width 0.25) (layer B.Cu) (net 7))
 (segment (start 172.5537 137.5188) (end 171.2155 137.5188) (width 0.25) (layer B.Cu) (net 7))
 (segment (start 171.2155 137.5188) (end 171.2155 137.5189) (width 0.25) (layer B.Cu) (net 7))
 (via (at 171.2155 137.5189) (size 0.8) (layers F.Cu B.Cu) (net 7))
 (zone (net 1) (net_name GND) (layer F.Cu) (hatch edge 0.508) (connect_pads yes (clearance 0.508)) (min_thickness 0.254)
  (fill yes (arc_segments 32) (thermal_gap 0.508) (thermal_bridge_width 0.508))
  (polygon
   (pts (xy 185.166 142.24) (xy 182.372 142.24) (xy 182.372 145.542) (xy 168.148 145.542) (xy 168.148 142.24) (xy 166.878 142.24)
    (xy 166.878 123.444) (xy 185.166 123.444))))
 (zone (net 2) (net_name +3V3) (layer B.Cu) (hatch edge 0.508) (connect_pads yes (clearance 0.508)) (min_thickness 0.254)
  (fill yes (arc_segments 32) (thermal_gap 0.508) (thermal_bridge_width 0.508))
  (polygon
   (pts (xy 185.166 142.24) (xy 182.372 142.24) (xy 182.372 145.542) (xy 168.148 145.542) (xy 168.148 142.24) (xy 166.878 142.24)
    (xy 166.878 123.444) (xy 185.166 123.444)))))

